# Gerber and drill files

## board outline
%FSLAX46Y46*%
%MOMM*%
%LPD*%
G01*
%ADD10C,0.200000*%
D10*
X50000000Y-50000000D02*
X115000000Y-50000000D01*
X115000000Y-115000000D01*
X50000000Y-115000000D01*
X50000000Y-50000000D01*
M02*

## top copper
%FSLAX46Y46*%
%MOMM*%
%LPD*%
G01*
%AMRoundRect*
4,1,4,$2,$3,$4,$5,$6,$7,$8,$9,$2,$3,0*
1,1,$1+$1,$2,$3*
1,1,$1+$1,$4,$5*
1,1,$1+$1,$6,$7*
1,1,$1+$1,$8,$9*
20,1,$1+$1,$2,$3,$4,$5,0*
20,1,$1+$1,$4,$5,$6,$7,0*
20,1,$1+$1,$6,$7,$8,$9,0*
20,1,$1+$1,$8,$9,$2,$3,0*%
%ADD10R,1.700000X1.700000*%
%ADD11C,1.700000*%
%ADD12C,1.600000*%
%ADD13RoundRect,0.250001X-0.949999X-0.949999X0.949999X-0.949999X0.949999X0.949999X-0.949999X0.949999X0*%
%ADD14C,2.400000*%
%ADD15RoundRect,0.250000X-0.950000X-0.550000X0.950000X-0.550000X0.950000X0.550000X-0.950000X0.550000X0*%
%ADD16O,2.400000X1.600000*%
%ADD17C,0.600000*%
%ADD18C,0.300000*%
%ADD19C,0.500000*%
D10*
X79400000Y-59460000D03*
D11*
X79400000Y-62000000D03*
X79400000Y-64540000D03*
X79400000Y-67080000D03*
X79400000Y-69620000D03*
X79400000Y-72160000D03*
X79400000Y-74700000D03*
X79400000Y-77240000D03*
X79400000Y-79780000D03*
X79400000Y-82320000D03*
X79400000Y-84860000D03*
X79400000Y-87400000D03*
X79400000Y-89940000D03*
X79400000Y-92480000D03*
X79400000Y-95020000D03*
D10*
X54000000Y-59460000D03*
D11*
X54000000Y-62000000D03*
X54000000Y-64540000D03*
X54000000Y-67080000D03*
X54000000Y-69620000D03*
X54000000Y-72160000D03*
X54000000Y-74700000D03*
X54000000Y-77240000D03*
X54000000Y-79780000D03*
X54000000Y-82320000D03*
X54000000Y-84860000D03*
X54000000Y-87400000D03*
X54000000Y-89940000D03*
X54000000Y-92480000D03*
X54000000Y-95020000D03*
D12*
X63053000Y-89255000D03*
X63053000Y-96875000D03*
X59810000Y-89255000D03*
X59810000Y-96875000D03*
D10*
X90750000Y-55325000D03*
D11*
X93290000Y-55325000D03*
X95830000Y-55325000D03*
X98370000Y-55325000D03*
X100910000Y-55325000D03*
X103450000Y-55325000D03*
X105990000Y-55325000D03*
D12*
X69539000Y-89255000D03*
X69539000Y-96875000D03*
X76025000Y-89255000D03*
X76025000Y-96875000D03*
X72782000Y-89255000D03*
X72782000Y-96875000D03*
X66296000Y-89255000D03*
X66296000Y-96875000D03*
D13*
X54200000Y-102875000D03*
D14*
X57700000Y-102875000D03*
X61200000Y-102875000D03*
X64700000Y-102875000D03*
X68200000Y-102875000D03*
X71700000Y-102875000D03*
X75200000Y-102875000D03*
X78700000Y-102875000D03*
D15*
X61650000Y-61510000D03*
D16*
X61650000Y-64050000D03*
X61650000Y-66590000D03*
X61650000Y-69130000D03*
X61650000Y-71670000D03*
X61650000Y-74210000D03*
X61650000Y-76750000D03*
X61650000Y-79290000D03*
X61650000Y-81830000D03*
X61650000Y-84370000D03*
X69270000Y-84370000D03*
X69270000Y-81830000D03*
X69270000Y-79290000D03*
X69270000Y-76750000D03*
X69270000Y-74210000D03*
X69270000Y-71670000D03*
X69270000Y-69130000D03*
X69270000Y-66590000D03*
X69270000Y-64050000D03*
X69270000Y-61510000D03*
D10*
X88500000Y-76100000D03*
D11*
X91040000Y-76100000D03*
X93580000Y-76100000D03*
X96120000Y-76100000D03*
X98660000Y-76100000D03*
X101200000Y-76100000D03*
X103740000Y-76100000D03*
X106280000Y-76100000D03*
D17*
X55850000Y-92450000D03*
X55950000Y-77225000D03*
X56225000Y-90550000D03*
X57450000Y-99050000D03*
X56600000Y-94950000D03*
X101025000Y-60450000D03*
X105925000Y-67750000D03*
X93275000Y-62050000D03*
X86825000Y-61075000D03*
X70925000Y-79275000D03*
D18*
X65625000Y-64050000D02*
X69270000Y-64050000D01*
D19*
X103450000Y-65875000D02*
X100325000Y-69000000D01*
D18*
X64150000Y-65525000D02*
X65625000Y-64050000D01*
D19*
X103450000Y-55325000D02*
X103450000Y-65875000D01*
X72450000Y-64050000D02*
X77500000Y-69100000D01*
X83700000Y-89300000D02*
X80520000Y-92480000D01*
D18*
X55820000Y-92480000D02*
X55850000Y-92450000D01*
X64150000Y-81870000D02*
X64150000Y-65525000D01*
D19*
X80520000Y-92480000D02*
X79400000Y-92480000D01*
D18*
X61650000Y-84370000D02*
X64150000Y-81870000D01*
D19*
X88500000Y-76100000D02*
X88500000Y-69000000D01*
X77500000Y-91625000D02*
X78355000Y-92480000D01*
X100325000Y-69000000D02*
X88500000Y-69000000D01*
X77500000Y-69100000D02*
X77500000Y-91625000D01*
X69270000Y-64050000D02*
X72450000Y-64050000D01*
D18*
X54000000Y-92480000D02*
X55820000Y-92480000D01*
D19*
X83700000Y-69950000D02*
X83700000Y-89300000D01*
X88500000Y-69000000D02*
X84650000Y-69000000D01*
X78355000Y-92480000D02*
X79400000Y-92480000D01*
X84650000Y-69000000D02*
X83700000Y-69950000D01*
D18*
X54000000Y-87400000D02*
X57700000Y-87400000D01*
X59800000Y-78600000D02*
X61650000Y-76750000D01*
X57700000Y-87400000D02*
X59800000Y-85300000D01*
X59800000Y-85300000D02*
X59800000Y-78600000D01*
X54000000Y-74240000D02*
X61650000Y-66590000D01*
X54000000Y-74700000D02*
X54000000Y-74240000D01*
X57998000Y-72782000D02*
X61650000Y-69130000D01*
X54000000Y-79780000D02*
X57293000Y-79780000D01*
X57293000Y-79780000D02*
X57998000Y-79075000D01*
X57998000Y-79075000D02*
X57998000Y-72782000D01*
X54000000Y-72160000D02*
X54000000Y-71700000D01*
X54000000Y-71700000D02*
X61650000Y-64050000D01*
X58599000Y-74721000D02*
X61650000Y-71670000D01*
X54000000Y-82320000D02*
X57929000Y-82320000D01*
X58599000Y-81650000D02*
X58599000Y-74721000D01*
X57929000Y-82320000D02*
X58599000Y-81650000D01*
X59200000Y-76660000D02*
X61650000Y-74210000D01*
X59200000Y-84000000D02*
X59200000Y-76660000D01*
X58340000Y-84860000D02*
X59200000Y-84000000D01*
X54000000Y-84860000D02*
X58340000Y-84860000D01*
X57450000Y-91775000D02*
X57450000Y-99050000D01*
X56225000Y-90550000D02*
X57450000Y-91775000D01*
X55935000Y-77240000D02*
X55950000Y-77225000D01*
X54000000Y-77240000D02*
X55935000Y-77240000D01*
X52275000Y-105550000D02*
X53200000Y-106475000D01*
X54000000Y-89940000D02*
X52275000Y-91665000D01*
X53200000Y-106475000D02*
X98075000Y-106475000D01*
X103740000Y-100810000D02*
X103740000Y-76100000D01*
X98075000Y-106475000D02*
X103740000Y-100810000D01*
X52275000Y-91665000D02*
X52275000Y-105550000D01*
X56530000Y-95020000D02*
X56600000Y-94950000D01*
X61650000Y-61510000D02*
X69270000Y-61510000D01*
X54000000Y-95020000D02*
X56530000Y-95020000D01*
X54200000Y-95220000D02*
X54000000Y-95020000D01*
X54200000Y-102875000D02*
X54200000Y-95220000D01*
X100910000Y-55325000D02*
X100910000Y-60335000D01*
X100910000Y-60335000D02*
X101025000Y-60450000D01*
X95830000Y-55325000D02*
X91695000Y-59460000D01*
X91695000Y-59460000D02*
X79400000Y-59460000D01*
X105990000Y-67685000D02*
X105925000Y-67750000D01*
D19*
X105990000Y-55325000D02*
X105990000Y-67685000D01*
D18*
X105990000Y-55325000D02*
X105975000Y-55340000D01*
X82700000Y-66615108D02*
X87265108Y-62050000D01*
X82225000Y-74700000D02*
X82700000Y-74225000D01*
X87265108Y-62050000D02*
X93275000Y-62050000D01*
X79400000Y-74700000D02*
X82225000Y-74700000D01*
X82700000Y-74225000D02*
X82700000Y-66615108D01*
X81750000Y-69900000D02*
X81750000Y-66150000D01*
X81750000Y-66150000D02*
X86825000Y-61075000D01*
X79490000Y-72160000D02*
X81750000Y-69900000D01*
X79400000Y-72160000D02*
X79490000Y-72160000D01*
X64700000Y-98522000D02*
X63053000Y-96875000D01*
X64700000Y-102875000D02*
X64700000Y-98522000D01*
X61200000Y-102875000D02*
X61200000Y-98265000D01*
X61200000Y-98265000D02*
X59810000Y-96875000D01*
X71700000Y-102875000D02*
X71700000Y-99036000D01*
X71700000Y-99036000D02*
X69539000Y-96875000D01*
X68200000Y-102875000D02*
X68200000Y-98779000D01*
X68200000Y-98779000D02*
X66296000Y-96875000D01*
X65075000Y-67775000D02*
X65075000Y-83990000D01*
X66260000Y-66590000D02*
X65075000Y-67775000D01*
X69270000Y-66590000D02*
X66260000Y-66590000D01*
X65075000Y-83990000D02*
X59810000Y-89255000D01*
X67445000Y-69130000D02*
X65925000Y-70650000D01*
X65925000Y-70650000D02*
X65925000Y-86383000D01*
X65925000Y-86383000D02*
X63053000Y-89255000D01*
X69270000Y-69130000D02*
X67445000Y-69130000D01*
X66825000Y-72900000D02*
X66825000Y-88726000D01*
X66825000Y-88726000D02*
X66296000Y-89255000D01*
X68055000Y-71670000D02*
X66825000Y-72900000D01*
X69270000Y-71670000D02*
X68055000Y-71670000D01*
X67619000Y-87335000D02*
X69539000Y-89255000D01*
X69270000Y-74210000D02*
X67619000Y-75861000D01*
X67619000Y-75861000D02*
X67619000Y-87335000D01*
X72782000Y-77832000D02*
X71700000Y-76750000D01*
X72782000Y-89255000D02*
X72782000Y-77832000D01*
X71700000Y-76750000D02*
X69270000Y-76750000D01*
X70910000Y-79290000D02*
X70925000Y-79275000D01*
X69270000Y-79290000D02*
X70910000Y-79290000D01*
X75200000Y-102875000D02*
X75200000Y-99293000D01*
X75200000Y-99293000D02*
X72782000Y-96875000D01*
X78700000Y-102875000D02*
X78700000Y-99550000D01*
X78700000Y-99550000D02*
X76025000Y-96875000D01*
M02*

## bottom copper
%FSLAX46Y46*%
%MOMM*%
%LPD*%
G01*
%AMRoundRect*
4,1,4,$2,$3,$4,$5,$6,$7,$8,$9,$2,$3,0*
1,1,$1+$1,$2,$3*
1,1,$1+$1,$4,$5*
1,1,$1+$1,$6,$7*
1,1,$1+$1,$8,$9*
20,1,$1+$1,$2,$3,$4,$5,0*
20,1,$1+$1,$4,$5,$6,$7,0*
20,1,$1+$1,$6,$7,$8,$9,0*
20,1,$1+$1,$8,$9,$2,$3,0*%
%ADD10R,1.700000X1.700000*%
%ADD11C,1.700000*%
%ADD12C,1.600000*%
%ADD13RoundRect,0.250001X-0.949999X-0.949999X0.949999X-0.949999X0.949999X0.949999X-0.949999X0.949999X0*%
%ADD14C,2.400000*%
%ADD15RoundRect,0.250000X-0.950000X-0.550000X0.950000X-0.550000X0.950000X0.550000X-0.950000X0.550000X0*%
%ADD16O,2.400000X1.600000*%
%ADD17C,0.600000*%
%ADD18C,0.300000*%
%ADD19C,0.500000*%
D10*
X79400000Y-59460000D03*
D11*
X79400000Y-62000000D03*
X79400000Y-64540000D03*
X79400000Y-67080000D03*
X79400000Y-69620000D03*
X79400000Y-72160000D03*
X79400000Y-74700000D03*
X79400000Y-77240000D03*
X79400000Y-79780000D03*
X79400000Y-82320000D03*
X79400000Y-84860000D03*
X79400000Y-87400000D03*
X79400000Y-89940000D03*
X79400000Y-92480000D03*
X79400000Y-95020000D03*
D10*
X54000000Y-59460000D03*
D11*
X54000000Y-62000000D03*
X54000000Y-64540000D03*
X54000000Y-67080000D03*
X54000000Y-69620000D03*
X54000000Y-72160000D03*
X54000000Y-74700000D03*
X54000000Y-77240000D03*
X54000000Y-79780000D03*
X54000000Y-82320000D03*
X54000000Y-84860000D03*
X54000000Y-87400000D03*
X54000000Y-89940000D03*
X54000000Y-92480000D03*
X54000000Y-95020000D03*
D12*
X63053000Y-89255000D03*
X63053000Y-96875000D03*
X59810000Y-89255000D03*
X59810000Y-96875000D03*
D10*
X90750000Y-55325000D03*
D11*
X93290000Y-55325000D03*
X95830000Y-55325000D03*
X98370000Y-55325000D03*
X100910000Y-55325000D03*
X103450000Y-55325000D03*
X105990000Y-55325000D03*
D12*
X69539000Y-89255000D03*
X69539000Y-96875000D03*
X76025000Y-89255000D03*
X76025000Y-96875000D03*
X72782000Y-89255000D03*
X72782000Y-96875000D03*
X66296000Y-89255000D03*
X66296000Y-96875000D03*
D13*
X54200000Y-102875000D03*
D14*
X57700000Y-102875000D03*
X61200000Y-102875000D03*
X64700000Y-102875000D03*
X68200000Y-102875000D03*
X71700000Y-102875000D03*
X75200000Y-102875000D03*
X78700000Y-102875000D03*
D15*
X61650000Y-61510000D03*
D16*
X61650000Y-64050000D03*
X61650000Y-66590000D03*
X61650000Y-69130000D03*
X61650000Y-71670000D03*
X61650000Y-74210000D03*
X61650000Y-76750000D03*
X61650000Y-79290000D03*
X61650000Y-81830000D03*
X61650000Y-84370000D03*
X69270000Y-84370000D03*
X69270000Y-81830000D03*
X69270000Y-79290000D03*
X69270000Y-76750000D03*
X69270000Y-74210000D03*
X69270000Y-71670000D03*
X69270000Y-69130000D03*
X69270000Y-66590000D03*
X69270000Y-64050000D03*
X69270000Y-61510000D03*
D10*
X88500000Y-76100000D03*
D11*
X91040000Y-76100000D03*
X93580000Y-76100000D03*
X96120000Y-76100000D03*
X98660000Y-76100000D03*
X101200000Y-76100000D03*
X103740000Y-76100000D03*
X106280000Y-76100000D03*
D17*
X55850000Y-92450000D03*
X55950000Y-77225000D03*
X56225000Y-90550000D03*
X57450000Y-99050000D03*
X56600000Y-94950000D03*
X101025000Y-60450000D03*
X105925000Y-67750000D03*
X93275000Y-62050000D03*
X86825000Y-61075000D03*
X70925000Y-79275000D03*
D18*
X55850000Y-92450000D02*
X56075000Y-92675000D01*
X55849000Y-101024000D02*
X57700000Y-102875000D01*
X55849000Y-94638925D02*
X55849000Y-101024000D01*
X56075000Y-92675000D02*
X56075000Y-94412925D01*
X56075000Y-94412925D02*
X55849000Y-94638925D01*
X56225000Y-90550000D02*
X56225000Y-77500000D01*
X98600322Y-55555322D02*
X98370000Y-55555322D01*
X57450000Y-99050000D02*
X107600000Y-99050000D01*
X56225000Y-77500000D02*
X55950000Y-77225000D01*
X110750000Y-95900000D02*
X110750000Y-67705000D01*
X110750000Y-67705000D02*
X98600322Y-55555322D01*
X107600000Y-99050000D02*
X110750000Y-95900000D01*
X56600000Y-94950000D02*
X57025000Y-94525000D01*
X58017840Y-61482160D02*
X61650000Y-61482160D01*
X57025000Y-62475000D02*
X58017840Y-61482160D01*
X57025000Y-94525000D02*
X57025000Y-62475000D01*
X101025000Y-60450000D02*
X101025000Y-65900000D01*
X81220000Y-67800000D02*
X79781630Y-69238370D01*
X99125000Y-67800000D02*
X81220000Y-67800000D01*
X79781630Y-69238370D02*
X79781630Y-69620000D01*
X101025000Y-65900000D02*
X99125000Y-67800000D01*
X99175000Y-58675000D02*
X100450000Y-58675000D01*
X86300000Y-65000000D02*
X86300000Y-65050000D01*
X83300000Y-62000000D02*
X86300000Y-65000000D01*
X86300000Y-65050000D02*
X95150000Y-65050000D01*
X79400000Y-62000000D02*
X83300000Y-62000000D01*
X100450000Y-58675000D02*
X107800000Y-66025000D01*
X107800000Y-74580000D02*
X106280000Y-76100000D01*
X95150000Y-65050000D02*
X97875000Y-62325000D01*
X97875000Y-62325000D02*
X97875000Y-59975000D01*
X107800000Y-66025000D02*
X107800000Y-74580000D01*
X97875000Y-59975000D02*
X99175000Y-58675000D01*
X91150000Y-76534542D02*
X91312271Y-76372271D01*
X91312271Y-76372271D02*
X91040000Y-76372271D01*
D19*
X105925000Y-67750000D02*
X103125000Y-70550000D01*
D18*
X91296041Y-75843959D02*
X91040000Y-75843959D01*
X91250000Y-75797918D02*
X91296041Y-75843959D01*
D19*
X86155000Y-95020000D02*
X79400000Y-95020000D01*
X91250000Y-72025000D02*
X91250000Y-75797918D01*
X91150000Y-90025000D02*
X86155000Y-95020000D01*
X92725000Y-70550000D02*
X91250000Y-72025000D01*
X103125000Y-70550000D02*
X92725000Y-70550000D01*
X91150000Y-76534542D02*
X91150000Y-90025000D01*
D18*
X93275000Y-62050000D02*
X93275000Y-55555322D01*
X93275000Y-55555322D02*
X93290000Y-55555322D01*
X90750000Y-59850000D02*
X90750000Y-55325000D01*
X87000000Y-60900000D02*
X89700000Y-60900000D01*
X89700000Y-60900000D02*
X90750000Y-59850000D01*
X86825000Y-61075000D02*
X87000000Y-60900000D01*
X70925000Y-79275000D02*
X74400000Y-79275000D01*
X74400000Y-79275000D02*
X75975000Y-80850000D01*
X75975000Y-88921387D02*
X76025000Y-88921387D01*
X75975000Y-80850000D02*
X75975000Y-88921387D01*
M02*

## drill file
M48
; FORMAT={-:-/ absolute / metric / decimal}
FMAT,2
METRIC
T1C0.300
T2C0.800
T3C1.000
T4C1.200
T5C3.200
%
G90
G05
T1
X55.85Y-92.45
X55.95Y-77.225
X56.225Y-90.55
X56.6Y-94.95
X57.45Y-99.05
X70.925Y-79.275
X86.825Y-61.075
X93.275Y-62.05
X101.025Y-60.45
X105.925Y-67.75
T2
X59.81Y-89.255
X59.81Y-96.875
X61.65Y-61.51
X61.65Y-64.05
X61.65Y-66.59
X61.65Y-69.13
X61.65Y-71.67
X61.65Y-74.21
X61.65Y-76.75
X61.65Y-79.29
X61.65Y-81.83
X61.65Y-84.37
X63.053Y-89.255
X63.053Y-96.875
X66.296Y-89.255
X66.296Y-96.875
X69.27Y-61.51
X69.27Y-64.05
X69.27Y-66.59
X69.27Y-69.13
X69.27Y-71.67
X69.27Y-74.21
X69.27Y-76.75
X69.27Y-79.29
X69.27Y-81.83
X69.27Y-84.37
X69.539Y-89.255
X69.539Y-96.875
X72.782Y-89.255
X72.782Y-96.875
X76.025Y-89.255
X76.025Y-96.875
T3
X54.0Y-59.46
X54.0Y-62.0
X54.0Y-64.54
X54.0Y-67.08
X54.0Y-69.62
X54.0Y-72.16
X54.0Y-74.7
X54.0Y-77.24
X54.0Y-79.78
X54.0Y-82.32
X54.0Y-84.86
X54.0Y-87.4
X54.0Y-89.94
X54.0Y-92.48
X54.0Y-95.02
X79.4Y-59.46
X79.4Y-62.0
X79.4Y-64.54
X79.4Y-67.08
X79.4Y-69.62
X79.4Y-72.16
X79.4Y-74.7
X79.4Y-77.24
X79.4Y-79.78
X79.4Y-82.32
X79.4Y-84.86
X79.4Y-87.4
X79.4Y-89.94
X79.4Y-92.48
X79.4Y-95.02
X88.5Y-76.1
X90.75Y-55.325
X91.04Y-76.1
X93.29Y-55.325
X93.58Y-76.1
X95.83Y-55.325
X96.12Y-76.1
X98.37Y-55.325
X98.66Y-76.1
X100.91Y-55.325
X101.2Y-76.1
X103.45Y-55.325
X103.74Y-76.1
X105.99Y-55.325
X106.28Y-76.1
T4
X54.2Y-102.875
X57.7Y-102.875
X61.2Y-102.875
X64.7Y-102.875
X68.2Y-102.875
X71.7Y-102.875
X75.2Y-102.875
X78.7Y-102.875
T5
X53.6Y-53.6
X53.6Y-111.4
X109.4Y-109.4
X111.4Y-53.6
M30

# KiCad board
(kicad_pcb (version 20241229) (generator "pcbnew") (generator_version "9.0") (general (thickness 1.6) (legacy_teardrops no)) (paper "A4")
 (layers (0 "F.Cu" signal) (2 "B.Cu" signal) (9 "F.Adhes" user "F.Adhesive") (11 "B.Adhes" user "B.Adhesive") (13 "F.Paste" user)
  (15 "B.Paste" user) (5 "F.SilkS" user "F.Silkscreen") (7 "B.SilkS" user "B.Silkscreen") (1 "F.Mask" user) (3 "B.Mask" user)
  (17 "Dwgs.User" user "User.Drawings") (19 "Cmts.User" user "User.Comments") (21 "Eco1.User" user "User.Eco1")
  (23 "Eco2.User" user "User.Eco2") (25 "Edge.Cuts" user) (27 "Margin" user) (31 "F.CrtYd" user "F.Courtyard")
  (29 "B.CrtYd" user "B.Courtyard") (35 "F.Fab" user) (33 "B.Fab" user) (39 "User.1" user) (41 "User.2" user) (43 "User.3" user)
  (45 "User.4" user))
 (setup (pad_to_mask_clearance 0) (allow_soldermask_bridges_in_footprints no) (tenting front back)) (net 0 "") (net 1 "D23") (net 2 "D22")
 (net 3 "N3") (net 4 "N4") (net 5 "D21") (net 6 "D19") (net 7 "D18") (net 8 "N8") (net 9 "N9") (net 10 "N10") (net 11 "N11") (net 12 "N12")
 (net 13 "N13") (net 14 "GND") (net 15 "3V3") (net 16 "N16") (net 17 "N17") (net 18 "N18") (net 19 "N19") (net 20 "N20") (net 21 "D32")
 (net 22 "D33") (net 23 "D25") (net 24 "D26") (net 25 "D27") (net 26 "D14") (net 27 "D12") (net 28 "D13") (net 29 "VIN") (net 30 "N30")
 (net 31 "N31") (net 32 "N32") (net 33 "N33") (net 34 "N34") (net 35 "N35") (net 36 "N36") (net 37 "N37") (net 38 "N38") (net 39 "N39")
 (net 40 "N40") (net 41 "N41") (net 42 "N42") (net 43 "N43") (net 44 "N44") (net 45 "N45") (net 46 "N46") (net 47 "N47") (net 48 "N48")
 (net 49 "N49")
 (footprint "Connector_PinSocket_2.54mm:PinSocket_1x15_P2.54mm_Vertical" (layer "F.Cu") (at 79.4 59.46)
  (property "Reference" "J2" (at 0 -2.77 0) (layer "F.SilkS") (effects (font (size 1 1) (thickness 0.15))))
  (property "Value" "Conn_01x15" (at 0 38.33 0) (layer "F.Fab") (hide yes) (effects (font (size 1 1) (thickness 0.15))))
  (pad "1" thru_hole rect (at 0 0) (size 1.7 1.7) (drill 1) (layers "*.Cu" "*.Mask") (remove_unused_layers no) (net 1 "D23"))
  (pad "2" thru_hole circle (at 0 2.54) (size 1.7 1.7) (drill 1) (layers "*.Cu" "*.Mask") (remove_unused_layers no) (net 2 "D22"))
  (pad "3" thru_hole circle (at 0 5.08) (size 1.7 1.7) (drill 1) (layers "*.Cu" "*.Mask") (remove_unused_layers no) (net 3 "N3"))
  (pad "4" thru_hole circle (at 0 7.62) (size 1.7 1.7) (drill 1) (layers "*.Cu" "*.Mask") (remove_unused_layers no) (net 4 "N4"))
  (pad "5" thru_hole circle (at 0 10.16) (size 1.7 1.7) (drill 1) (layers "*.Cu" "*.Mask") (remove_unused_layers no) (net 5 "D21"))
  (pad "6" thru_hole circle (at 0 12.7) (size 1.7 1.7) (drill 1) (layers "*.Cu" "*.Mask") (remove_unused_layers no) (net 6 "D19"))
  (pad "7" thru_hole circle (at 0 15.24) (size 1.7 1.7) (drill 1) (layers "*.Cu" "*.Mask") (remove_unused_layers no) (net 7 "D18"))
  (pad "8" thru_hole circle (at 0 17.78) (size 1.7 1.7) (drill 1) (layers "*.Cu" "*.Mask") (remove_unused_layers no) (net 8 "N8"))
  (pad "9" thru_hole circle (at 0 20.32) (size 1.7 1.7) (drill 1) (layers "*.Cu" "*.Mask") (remove_unused_layers no) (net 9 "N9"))
  (pad "10" thru_hole circle (at 0 22.86) (size 1.7 1.7) (drill 1) (layers "*.Cu" "*.Mask") (remove_unused_layers no) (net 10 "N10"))
  (pad "11" thru_hole circle (at 0 25.4) (size 1.7 1.7) (drill 1) (layers "*.Cu" "*.Mask") (remove_unused_layers no) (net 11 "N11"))
  (pad "12" thru_hole circle (at 0 27.94) (size 1.7 1.7) (drill 1) (layers "*.Cu" "*.Mask") (remove_unused_layers no) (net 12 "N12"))
  (pad "13" thru_hole circle (at 0 30.48) (size 1.7 1.7) (drill 1) (layers "*.Cu" "*.Mask") (remove_unused_layers no) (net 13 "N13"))
  (pad "14" thru_hole circle (at 0 33.02) (size 1.7 1.7) (drill 1) (layers "*.Cu" "*.Mask") (remove_unused_layers no) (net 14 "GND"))
  (pad "15" thru_hole circle (at 0 35.56) (size 1.7 1.7) (drill 1) (layers "*.Cu" "*.Mask") (remove_unused_layers no) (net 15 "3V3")))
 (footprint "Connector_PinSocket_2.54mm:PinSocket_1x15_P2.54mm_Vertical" (layer "F.Cu") (at 54 59.46)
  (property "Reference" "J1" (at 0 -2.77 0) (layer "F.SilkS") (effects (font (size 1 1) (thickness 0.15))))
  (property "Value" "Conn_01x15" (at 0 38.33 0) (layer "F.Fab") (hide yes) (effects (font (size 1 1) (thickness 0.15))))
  (pad "1" thru_hole rect (at 0 0) (size 1.7 1.7) (drill 1) (layers "*.Cu" "*.Mask") (remove_unused_layers no) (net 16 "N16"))
  (pad "2" thru_hole circle (at 0 2.54) (size 1.7 1.7) (drill 1) (layers "*.Cu" "*.Mask") (remove_unused_layers no) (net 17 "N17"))
  (pad "3" thru_hole circle (at 0 5.08) (size 1.7 1.7) (drill 1) (layers "*.Cu" "*.Mask") (remove_unused_layers no) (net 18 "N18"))
  (pad "4" thru_hole circle (at 0 7.62) (size 1.7 1.7) (drill 1) (layers "*.Cu" "*.Mask") (remove_unused_layers no) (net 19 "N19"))
  (pad "5" thru_hole circle (at 0 10.16) (size 1.7 1.7) (drill 1) (layers "*.Cu" "*.Mask") (remove_unused_layers no) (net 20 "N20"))
  (pad "6" thru_hole circle (at 0 12.7) (size 1.7 1.7) (drill 1) (layers "*.Cu" "*.Mask") (remove_unused_layers no) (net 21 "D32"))
  (pad "7" thru_hole circle (at 0 15.24) (size 1.7 1.7) (drill 1) (layers "*.Cu" "*.Mask") (remove_unused_layers no) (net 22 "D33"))
  (pad "8" thru_hole circle (at 0 17.78) (size 1.7 1.7) (drill 1) (layers "*.Cu" "*.Mask") (remove_unused_layers no) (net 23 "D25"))
  (pad "9" thru_hole circle (at 0 20.32) (size 1.7 1.7) (drill 1) (layers "*.Cu" "*.Mask") (remove_unused_layers no) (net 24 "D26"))
  (pad "10" thru_hole circle (at 0 22.86) (size 1.7 1.7) (drill 1) (layers "*.Cu" "*.Mask") (remove_unused_layers no) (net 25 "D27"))
  (pad "11" thru_hole circle (at 0 25.4) (size 1.7 1.7) (drill 1) (layers "*.Cu" "*.Mask") (remove_unused_layers no) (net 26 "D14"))
  (pad "12" thru_hole circle (at 0 27.94) (size 1.7 1.7) (drill 1) (layers "*.Cu" "*.Mask") (remove_unused_layers no) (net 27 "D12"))
  (pad "13" thru_hole circle (at 0 30.48) (size 1.7 1.7) (drill 1) (layers "*.Cu" "*.Mask") (remove_unused_layers no) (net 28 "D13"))
  (pad "14" thru_hole circle (at 0 33.02) (size 1.7 1.7) (drill 1) (layers "*.Cu" "*.Mask") (remove_unused_layers no) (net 14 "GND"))
  (pad "15" thru_hole circle (at 0 35.56) (size 1.7 1.7) (drill 1) (layers "*.Cu" "*.Mask") (remove_unused_layers no) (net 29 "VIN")))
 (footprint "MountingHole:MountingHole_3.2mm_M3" (layer "F.Cu") (at 53.6 53.6)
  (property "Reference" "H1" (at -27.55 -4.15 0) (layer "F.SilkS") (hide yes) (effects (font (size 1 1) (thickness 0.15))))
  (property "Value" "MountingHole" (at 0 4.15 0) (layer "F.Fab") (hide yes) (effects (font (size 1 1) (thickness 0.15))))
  (pad "" np_thru_hole circle (at 0 0) (size 3.2 3.2) (drill 3.2) (layers "*.Cu" "*.Mask")))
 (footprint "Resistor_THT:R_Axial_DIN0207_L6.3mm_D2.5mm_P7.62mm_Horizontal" (layer "F.Cu") (at 63.053 89.255 -90)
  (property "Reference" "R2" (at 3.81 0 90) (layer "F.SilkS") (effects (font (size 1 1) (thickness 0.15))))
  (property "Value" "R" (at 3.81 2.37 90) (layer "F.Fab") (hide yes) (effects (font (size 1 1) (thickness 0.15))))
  (pad "1" thru_hole circle (at 0 0 270) (size 1.6 1.6) (drill 0.8) (layers "*.Cu" "*.Mask") (remove_unused_layers no) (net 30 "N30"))
  (pad "2" thru_hole circle (at 7.62 0 270) (size 1.6 1.6) (drill 0.8) (layers "*.Cu" "*.Mask") (remove_unused_layers no) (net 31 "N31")))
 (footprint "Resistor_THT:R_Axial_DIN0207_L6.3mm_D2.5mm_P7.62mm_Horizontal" (layer "F.Cu") (at 59.81 89.255 -90)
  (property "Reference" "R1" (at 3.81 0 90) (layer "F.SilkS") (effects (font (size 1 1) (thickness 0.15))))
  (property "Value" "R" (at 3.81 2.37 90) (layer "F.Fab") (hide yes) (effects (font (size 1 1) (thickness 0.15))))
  (pad "1" thru_hole circle (at 0 0 270) (size 1.6 1.6) (drill 0.8) (layers "*.Cu" "*.Mask") (remove_unused_layers no) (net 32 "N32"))
  (pad "2" thru_hole circle (at 7.62 0 270) (size 1.6 1.6) (drill 0.8) (layers "*.Cu" "*.Mask") (remove_unused_layers no) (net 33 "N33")))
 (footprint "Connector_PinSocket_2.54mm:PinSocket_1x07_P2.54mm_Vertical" (layer "F.Cu") (at 90.75 55.325 90)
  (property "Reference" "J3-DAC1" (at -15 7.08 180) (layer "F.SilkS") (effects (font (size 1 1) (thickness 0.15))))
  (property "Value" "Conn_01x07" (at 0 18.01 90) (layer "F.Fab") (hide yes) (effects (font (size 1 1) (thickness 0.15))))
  (pad "1" thru_hole rect (at 0 0 90) (size 1.7 1.7) (drill 1) (layers "*.Cu" "*.Mask") (remove_unused_layers no) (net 6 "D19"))
  (pad "2" thru_hole circle (at 0 2.54 90) (size 1.7 1.7) (drill 1) (layers "*.Cu" "*.Mask") (remove_unused_layers no) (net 7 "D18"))
  (pad "3" thru_hole circle (at 0 5.08 90) (size 1.7 1.7) (drill 1) (layers "*.Cu" "*.Mask") (remove_unused_layers no) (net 1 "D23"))
  (pad "4" thru_hole circle (at 0 7.62 90) (size 1.7 1.7) (drill 1) (layers "*.Cu" "*.Mask") (remove_unused_layers no) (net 23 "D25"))
  (pad "5" thru_hole circle (at 0 10.16 90) (size 1.7 1.7) (drill 1) (layers "*.Cu" "*.Mask") (remove_unused_layers no) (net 5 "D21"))
  (pad "6" thru_hole circle (at 0 12.7 90) (size 1.7 1.7) (drill 1) (layers "*.Cu" "*.Mask") (remove_unused_layers no) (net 14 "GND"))
  (pad "7" thru_hole circle (at 0 15.24 90) (size 1.7 1.7) (drill 1) (layers "*.Cu" "*.Mask") (remove_unused_layers no) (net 15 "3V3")))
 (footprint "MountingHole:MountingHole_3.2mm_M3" (layer "F.Cu") (at 53.6 111.4)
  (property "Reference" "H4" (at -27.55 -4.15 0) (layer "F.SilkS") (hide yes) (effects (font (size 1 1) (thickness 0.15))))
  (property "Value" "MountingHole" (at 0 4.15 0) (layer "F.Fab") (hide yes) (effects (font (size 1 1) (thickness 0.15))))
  (pad "" np_thru_hole circle (at 0 0) (size 3.2 3.2) (drill 3.2) (layers "*.Cu" "*.Mask")))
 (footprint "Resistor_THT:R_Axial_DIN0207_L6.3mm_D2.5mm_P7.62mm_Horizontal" (layer "F.Cu") (at 69.539 89.255 -90)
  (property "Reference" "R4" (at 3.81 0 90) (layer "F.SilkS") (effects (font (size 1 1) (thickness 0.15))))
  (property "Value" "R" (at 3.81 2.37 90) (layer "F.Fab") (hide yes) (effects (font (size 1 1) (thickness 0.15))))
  (pad "1" thru_hole circle (at 0 0 270) (size 1.6 1.6) (drill 0.8) (layers "*.Cu" "*.Mask") (remove_unused_layers no) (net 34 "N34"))
  (pad "2" thru_hole circle (at 7.62 0 270) (size 1.6 1.6) (drill 0.8) (layers "*.Cu" "*.Mask") (remove_unused_layers no) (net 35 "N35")))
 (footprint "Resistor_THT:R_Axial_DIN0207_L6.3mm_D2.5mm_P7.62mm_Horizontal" (layer "F.Cu") (at 76.025 89.255 -90)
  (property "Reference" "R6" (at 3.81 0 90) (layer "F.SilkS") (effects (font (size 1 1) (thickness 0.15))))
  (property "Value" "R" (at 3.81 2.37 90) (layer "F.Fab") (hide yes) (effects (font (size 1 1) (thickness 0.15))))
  (pad "1" thru_hole circle (at 0 0 270) (size 1.6 1.6) (drill 0.8) (layers "*.Cu" "*.Mask") (remove_unused_layers no) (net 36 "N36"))
  (pad "2" thru_hole circle (at 7.62 0 270) (size 1.6 1.6) (drill 0.8) (layers "*.Cu" "*.Mask") (remove_unused_layers no) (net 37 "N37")))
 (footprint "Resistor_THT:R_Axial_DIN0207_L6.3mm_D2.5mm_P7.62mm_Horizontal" (layer "F.Cu") (at 72.782 89.255 -90)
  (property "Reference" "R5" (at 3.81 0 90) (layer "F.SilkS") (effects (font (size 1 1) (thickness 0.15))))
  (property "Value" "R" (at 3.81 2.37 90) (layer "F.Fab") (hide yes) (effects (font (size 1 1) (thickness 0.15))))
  (pad "1" thru_hole circle (at 0 0 270) (size 1.6 1.6) (drill 0.8) (layers "*.Cu" "*.Mask") (remove_unused_layers no) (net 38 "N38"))
  (pad "2" thru_hole circle (at 7.62 0 270) (size 1.6 1.6) (drill 0.8) (layers "*.Cu" "*.Mask") (remove_unused_layers no) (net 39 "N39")))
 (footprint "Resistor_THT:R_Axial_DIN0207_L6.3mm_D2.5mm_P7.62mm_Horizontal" (layer "F.Cu") (at 66.296 89.255 -90)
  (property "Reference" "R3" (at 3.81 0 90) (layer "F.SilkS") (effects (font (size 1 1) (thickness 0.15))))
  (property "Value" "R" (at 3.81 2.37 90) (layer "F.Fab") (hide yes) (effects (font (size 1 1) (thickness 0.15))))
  (pad "1" thru_hole circle (at 0 0 270) (size 1.6 1.6) (drill 0.8) (layers "*.Cu" "*.Mask") (remove_unused_layers no) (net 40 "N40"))
  (pad "2" thru_hole circle (at 7.62 0 270) (size 1.6 1.6) (drill 0.8) (layers "*.Cu" "*.Mask") (remove_unused_layers no) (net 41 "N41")))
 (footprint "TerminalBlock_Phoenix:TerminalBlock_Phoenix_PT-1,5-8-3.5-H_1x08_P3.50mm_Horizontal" (layer "F.Cu") (at 54.2 102.875)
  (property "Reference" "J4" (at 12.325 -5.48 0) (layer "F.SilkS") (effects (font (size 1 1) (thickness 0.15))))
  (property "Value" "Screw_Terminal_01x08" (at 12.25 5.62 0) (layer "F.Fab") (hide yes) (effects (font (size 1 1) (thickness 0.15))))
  (pad "1" thru_hole roundrect (at 0 0) (size 2.4 2.4) (drill 1.2) (layers "*.Cu" "*.Mask") (remove_unused_layers no)
   (roundrect_rratio 0.104167) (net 29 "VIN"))
  (pad "2" thru_hole circle (at 3.5 0) (size 2.4 2.4) (drill 1.2) (layers "*.Cu" "*.Mask") (remove_unused_layers no) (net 14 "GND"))
  (pad "3" thru_hole circle (at 7 0) (size 2.4 2.4) (drill 1.2) (layers "*.Cu" "*.Mask") (remove_unused_layers no) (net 33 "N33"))
  (pad "4" thru_hole circle (at 10.5 0) (size 2.4 2.4) (drill 1.2) (layers "*.Cu" "*.Mask") (remove_unused_layers no) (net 31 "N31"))
  (pad "5" thru_hole circle (at 14 0) (size 2.4 2.4) (drill 1.2) (layers "*.Cu" "*.Mask") (remove_unused_layers no) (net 41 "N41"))
  (pad "6" thru_hole circle (at 17.5 0) (size 2.4 2.4) (drill 1.2) (layers "*.Cu" "*.Mask") (remove_unused_layers no) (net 35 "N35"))
  (pad "7" thru_hole circle (at 21 0) (size 2.4 2.4) (drill 1.2) (layers "*.Cu" "*.Mask") (remove_unused_layers no) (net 39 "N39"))
  (pad "8" thru_hole circle (at 24.5 0) (size 2.4 2.4) (drill 1.2) (layers "*.Cu" "*.Mask") (remove_unused_layers no) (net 37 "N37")))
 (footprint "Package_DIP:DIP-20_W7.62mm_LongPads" (layer "F.Cu") (at 61.65 61.51)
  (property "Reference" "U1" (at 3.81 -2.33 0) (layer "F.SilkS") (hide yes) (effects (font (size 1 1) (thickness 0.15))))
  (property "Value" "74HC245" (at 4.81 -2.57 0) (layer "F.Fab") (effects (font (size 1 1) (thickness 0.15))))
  (pad "1" thru_hole roundrect (at 0 0) (size 2.4 1.6) (drill 0.8) (layers "*.Cu" "*.Mask") (remove_unused_layers no)
   (roundrect_rratio 0.15625) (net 29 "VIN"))
  (pad "2" thru_hole oval (at 0 2.54) (size 2.4 1.6) (drill 0.8) (layers "*.Cu" "*.Mask") (remove_unused_layers no) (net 21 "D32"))
  (pad "3" thru_hole oval (at 0 5.08) (size 2.4 1.6) (drill 0.8) (layers "*.Cu" "*.Mask") (remove_unused_layers no) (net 22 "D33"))
  (pad "4" thru_hole oval (at 0 7.62) (size 2.4 1.6) (drill 0.8) (layers "*.Cu" "*.Mask") (remove_unused_layers no) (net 24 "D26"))
  (pad "5" thru_hole oval (at 0 10.16) (size 2.4 1.6) (drill 0.8) (layers "*.Cu" "*.Mask") (remove_unused_layers no) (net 25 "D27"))
  (pad "6" thru_hole oval (at 0 12.7) (size 2.4 1.6) (drill 0.8) (layers "*.Cu" "*.Mask") (remove_unused_layers no) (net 26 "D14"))
  (pad "7" thru_hole oval (at 0 15.24) (size 2.4 1.6) (drill 0.8) (layers "*.Cu" "*.Mask") (remove_unused_layers no) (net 27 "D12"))
  (pad "8" thru_hole oval (at 0 17.78) (size 2.4 1.6) (drill 0.8) (layers "*.Cu" "*.Mask") (remove_unused_layers no) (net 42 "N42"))
  (pad "9" thru_hole oval (at 0 20.32) (size 2.4 1.6) (drill 0.8) (layers "*.Cu" "*.Mask") (remove_unused_layers no) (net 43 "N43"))
  (pad "10" thru_hole oval (at 0 22.86) (size 2.4 1.6) (drill 0.8) (layers "*.Cu" "*.Mask") (remove_unused_layers no) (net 14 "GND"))
  (pad "11" thru_hole oval (at 7.62 22.86) (size 2.4 1.6) (drill 0.8) (layers "*.Cu" "*.Mask") (remove_unused_layers no) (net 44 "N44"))
  (pad "12" thru_hole oval (at 7.62 20.32) (size 2.4 1.6) (drill 0.8) (layers "*.Cu" "*.Mask") (remove_unused_layers no) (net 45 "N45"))
  (pad "13" thru_hole oval (at 7.62 17.78) (size 2.4 1.6) (drill 0.8) (layers "*.Cu" "*.Mask") (remove_unused_layers no) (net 36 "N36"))
  (pad "14" thru_hole oval (at 7.62 15.24) (size 2.4 1.6) (drill 0.8) (layers "*.Cu" "*.Mask") (remove_unused_layers no) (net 38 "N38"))
  (pad "15" thru_hole oval (at 7.62 12.7) (size 2.4 1.6) (drill 0.8) (layers "*.Cu" "*.Mask") (remove_unused_layers no) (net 34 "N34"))
  (pad "16" thru_hole oval (at 7.62 10.16) (size 2.4 1.6) (drill 0.8) (layers "*.Cu" "*.Mask") (remove_unused_layers no) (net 40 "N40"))
  (pad "17" thru_hole oval (at 7.62 7.62) (size 2.4 1.6) (drill 0.8) (layers "*.Cu" "*.Mask") (remove_unused_layers no) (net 30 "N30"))
  (pad "18" thru_hole oval (at 7.62 5.08) (size 2.4 1.6) (drill 0.8) (layers "*.Cu" "*.Mask") (remove_unused_layers no) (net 32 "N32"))
  (pad "19" thru_hole oval (at 7.62 2.54) (size 2.4 1.6) (drill 0.8) (layers "*.Cu" "*.Mask") (remove_unused_layers no) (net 14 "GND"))
  (pad "20" thru_hole oval (at 7.62 0) (size 2.4 1.6) (drill 0.8) (layers "*.Cu" "*.Mask") (remove_unused_layers no) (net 29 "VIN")))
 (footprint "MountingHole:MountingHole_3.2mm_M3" (layer "F.Cu") (at 109.4 109.4)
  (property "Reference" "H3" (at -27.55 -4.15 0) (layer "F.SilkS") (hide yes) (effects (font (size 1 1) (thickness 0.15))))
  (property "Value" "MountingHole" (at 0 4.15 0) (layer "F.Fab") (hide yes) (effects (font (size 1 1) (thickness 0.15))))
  (pad "" np_thru_hole circle (at 0 0) (size 3.2 3.2) (drill 3.2) (layers "*.Cu" "*.Mask")))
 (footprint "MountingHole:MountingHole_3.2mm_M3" (layer "F.Cu") (at 111.4 53.6)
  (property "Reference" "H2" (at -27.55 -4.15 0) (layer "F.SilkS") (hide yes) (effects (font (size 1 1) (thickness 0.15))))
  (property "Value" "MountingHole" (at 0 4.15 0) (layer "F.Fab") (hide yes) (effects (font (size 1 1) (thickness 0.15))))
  (pad "" np_thru_hole circle (at 0 0) (size 3.2 3.2) (drill 3.2) (layers "*.Cu" "*.Mask")))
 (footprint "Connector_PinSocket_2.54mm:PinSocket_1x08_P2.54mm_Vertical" (layer "F.Cu") (at 88.5 76.1 90)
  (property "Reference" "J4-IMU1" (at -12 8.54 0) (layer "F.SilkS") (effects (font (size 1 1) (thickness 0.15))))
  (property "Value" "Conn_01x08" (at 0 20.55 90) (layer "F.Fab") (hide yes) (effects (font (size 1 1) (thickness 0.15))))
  (pad "1" thru_hole rect (at 0 0 90) (size 1.7 1.7) (drill 1) (layers "*.Cu" "*.Mask") (remove_unused_layers no) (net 14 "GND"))
  (pad "2" thru_hole circle (at 0 2.54 90) (size 1.7 1.7) (drill 1) (layers "*.Cu" "*.Mask") (remove_unused_layers no) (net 15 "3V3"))
  (pad "3" thru_hole circle (at 0 5.08 90) (size 1.7 1.7) (drill 1) (layers "*.Cu" "*.Mask") (remove_unused_layers no) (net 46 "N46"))
  (pad "4" thru_hole circle (at 0 7.62 90) (size 1.7 1.7) (drill 1) (layers "*.Cu" "*.Mask") (remove_unused_layers no) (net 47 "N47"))
  (pad "5" thru_hole circle (at 0 10.16 90) (size 1.7 1.7) (drill 1) (layers "*.Cu" "*.Mask") (remove_unused_layers no) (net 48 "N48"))
  (pad "6" thru_hole circle (at 0 12.7 90) (size 1.7 1.7) (drill 1) (layers "*.Cu" "*.Mask") (remove_unused_layers no) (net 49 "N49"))
  (pad "7" thru_hole circle (at 0 15.24 90) (size 1.7 1.7) (drill 1) (layers "*.Cu" "*.Mask") (remove_unused_layers no) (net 28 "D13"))
  (pad "8" thru_hole circle (at 0 17.78 90) (size 1.7 1.7) (drill 1) (layers "*.Cu" "*.Mask") (remove_unused_layers no) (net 2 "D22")))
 (gr_rect (start 50 50) (end 115 115) (stroke (width 0.2) (type solid)) (fill no) (layer "Edge.Cuts"))
 (segment (start 65.625 64.05) (end 69.27 64.05) (width 0.3) (layer "F.Cu") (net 14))
 (segment (start 103.45 65.875) (end 100.325 69) (width 0.5) (layer "F.Cu") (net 14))
 (segment (start 64.15 65.525) (end 65.625 64.05) (width 0.3) (layer "F.Cu") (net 14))
 (segment (start 103.45 55.325) (end 103.45 65.875) (width 0.5) (layer "F.Cu") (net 14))
 (segment (start 72.45 64.05) (end 77.5 69.1) (width 0.5) (layer "F.Cu") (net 14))
 (segment (start 83.7 89.3) (end 80.52 92.48) (width 0.5) (layer "F.Cu") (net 14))
 (segment (start 55.82 92.48) (end 55.85 92.45) (width 0.3) (layer "F.Cu") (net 14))
 (segment (start 64.15 81.87) (end 64.15 65.525) (width 0.3) (layer "F.Cu") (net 14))
 (segment (start 80.52 92.48) (end 79.4 92.48) (width 0.5) (layer "F.Cu") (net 14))
 (segment (start 61.65 84.37) (end 64.15 81.87) (width 0.3) (layer "F.Cu") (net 14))
 (segment (start 88.5 76.1) (end 88.5 69) (width 0.5) (layer "F.Cu") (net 14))
 (segment (start 77.5 91.625) (end 78.355 92.48) (width 0.5) (layer "F.Cu") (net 14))
 (segment (start 100.325 69) (end 88.5 69) (width 0.5) (layer "F.Cu") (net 14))
 (segment (start 77.5 69.1) (end 77.5 91.625) (width 0.5) (layer "F.Cu") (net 14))
 (segment (start 69.27 64.05) (end 72.45 64.05) (width 0.5) (layer "F.Cu") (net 14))
 (segment (start 54 92.48) (end 55.82 92.48) (width 0.3) (layer "F.Cu") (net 14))
 (segment (start 83.7 69.95) (end 83.7 89.3) (width 0.5) (layer "F.Cu") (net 14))
 (segment (start 88.5 69) (end 84.65 69) (width 0.5) (layer "F.Cu") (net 14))
 (segment (start 78.355 92.48) (end 79.4 92.48) (width 0.5) (layer "F.Cu") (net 14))
 (segment (start 84.65 69) (end 83.7 69.95) (width 0.5) (layer "F.Cu") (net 14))
 (via (at 55.85 92.45) (size 0.6) (drill 0.3) (layers "F.Cu" "B.Cu") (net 14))
 (segment (start 55.85 92.45) (end 56.075 92.675) (width 0.3) (layer "B.Cu") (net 14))
 (segment (start 55.849 101.024) (end 57.7 102.875) (width 0.3) (layer "B.Cu") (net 14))
 (segment (start 55.849 94.638925) (end 55.849 101.024) (width 0.3) (layer "B.Cu") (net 14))
 (segment (start 56.075 92.675) (end 56.075 94.412925) (width 0.3) (layer "B.Cu") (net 14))
 (segment (start 56.075 94.412925) (end 55.849 94.638925) (width 0.3) (layer "B.Cu") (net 14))
 (segment (start 54 87.4) (end 57.7 87.4) (width 0.3) (layer "F.Cu") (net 27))
 (segment (start 59.8 78.6) (end 61.65 76.75) (width 0.3) (layer "F.Cu") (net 27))
 (segment (start 57.7 87.4) (end 59.8 85.3) (width 0.3) (layer "F.Cu") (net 27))
 (segment (start 59.8 85.3) (end 59.8 78.6) (width 0.3) (layer "F.Cu") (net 27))
 (segment (start 54 74.24) (end 61.65 66.59) (width 0.3) (layer "F.Cu") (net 22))
 (segment (start 54 74.7) (end 54 74.24) (width 0.3) (layer "F.Cu") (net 22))
 (segment (start 57.998 72.782) (end 61.65 69.13) (width 0.3) (layer "F.Cu") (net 24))
 (segment (start 54 79.78) (end 57.293 79.78) (width 0.3) (layer "F.Cu") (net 24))
 (segment (start 57.293 79.78) (end 57.998 79.075) (width 0.3) (layer "F.Cu") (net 24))
 (segment (start 57.998 79.075) (end 57.998 72.782) (width 0.3) (layer "F.Cu") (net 24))
 (segment (start 54 72.16) (end 54 71.7) (width 0.3) (layer "F.Cu") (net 21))
 (segment (start 54 71.7) (end 61.65 64.05) (width 0.3) (layer "F.Cu") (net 21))
 (segment (start 58.599 74.721) (end 61.65 71.67) (width 0.3) (layer "F.Cu") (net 25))
 (segment (start 54 82.32) (end 57.929 82.32) (width 0.3) (layer "F.Cu") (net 25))
 (segment (start 58.599 81.65) (end 58.599 74.721) (width 0.3) (layer "F.Cu") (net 25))
 (segment (start 57.929 82.32) (end 58.599 81.65) (width 0.3) (layer "F.Cu") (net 25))
 (segment (start 59.2 76.66) (end 61.65 74.21) (width 0.3) (layer "F.Cu") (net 26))
 (segment (start 59.2 84) (end 59.2 76.66) (width 0.3) (layer "F.Cu") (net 26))
 (segment (start 58.34 84.86) (end 59.2 84) (width 0.3) (layer "F.Cu") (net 26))
 (segment (start 54 84.86) (end 58.34 84.86) (width 0.3) (layer "F.Cu") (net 26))
 (segment (start 57.45 91.775) (end 57.45 99.05) (width 0.3) (layer "F.Cu") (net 23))
 (segment (start 56.225 90.55) (end 57.45 91.775) (width 0.3) (layer "F.Cu") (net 23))
 (segment (start 55.935 77.24) (end 55.95 77.225) (width 0.3) (layer "F.Cu") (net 23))
 (segment (start 54 77.24) (end 55.935 77.24) (width 0.3) (layer "F.Cu") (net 23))
 (via (at 55.95 77.225) (size 0.6) (drill 0.3) (layers "F.Cu" "B.Cu") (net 23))
 (via (at 56.225 90.55) (size 0.6) (drill 0.3) (layers "F.Cu" "B.Cu") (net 23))
 (via (at 57.45 99.05) (size 0.6) (drill 0.3) (layers "F.Cu" "B.Cu") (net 23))
 (segment (start 56.225 90.55) (end 56.225 77.5) (width 0.3) (layer "B.Cu") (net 23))
 (segment (start 98.600322 55.555322) (end 98.37 55.555322) (width 0.3) (layer "B.Cu") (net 23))
 (segment (start 57.45 99.05) (end 107.6 99.05) (width 0.3) (layer "B.Cu") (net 23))
 (segment (start 56.225 77.5) (end 55.95 77.225) (width 0.3) (layer "B.Cu") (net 23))
 (segment (start 110.75 95.9) (end 110.75 67.705) (width 0.3) (layer "B.Cu") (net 23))
 (segment (start 110.75 67.705) (end 98.600322 55.555322) (width 0.3) (layer "B.Cu") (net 23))
 (segment (start 107.6 99.05) (end 110.75 95.9) (width 0.3) (layer "B.Cu") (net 23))
 (segment (start 52.275 105.55) (end 53.2 106.475) (width 0.3) (layer "F.Cu") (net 28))
 (segment (start 54 89.94) (end 52.275 91.665) (width 0.3) (layer "F.Cu") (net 28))
 (segment (start 53.2 106.475) (end 98.075 106.475) (width 0.3) (layer "F.Cu") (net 28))
 (segment (start 103.74 100.81) (end 103.74 76.1) (width 0.3) (layer "F.Cu") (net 28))
 (segment (start 98.075 106.475) (end 103.74 100.81) (width 0.3) (layer "F.Cu") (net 28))
 (segment (start 52.275 91.665) (end 52.275 105.55) (width 0.3) (layer "F.Cu") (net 28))
 (segment (start 56.53 95.02) (end 56.6 94.95) (width 0.3) (layer "F.Cu") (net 29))
 (segment (start 61.65 61.51) (end 69.27 61.51) (width 0.3) (layer "F.Cu") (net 29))
 (segment (start 54 95.02) (end 56.53 95.02) (width 0.3) (layer "F.Cu") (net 29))
 (segment (start 54.2 95.22) (end 54 95.02) (width 0.3) (layer "F.Cu") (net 29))
 (segment (start 54.2 102.875) (end 54.2 95.22) (width 0.3) (layer "F.Cu") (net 29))
 (via (at 56.6 94.95) (size 0.6) (drill 0.3) (layers "F.Cu" "B.Cu") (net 29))
 (segment (start 56.6 94.95) (end 57.025 94.525) (width 0.3) (layer "B.Cu") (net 29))
 (segment (start 58.01784 61.48216) (end 61.65 61.48216) (width 0.3) (layer "B.Cu") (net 29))
 (segment (start 57.025 62.475) (end 58.01784 61.48216) (width 0.3) (layer "B.Cu") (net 29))
 (segment (start 57.025 94.525) (end 57.025 62.475) (width 0.3) (layer "B.Cu") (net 29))
 (segment (start 100.91 55.325) (end 100.91 60.335) (width 0.3) (layer "F.Cu") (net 5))
 (segment (start 100.91 60.335) (end 101.025 60.45) (width 0.3) (layer "F.Cu") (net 5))
 (via (at 101.025 60.45) (size 0.6) (drill 0.3) (layers "F.Cu" "B.Cu") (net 5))
 (segment (start 101.025 60.45) (end 101.025 65.9) (width 0.3) (layer "B.Cu") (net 5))
 (segment (start 81.22 67.8) (end 79.78163 69.23837) (width 0.3) (layer "B.Cu") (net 5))
 (segment (start 99.125 67.8) (end 81.22 67.8) (width 0.3) (layer "B.Cu") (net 5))
 (segment (start 79.78163 69.23837) (end 79.78163 69.62) (width 0.3) (layer "B.Cu") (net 5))
 (segment (start 101.025 65.9) (end 99.125 67.8) (width 0.3) (layer "B.Cu") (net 5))
 (segment (start 95.83 55.325) (end 91.695 59.46) (width 0.3) (layer "F.Cu") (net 1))
 (segment (start 91.695 59.46) (end 79.4 59.46) (width 0.3) (layer "F.Cu") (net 1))
 (segment (start 99.175 58.675) (end 100.45 58.675) (width 0.3) (layer "B.Cu") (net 2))
 (segment (start 86.3 65) (end 86.3 65.05) (width 0.3) (layer "B.Cu") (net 2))
 (segment (start 83.3 62) (end 86.3 65) (width 0.3) (layer "B.Cu") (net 2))
 (segment (start 86.3 65.05) (end 95.15 65.05) (width 0.3) (layer "B.Cu") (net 2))
 (segment (start 79.4 62) (end 83.3 62) (width 0.3) (layer "B.Cu") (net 2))
 (segment (start 100.45 58.675) (end 107.8 66.025) (width 0.3) (layer "B.Cu") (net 2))
 (segment (start 107.8 74.58) (end 106.28 76.1) (width 0.3) (layer "B.Cu") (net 2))
 (segment (start 95.15 65.05) (end 97.875 62.325) (width 0.3) (layer "B.Cu") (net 2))
 (segment (start 97.875 62.325) (end 97.875 59.975) (width 0.3) (layer "B.Cu") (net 2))
 (segment (start 107.8 66.025) (end 107.8 74.58) (width 0.3) (layer "B.Cu") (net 2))
 (segment (start 97.875 59.975) (end 99.175 58.675) (width 0.3) (layer "B.Cu") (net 2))
 (segment (start 105.99 67.685) (end 105.925 67.75) (width 0.3) (layer "F.Cu") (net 15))
 (segment (start 105.99 55.325) (end 105.99 67.685) (width 0.5) (layer "F.Cu") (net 15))
 (segment (start 105.99 55.325) (end 105.975 55.34) (width 0.3) (layer "F.Cu") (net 15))
 (via (at 105.925 67.75) (size 0.6) (drill 0.3) (layers "F.Cu" "B.Cu") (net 15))
 (segment (start 91.15 76.534542) (end 91.312271 76.372271) (width 0.3) (layer "B.Cu") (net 15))
 (segment (start 91.312271 76.372271) (end 91.04 76.372271) (width 0.3) (layer "B.Cu") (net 15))
 (segment (start 105.925 67.75) (end 103.125 70.55) (width 0.5) (layer "B.Cu") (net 15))
 (segment (start 91.296041 75.843959) (end 91.04 75.843959) (width 0.3) (layer "B.Cu") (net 15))
 (segment (start 91.25 75.797918) (end 91.296041 75.843959) (width 0.3) (layer "B.Cu") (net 15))
 (segment (start 86.155 95.02) (end 79.4 95.02) (width 0.5) (layer "B.Cu") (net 15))
 (segment (start 91.25 72.025) (end 91.25 75.797918) (width 0.5) (layer "B.Cu") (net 15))
 (segment (start 91.15 90.025) (end 86.155 95.02) (width 0.5) (layer "B.Cu") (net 15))
 (segment (start 92.725 70.55) (end 91.25 72.025) (width 0.5) (layer "B.Cu") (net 15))
 (segment (start 103.125 70.55) (end 92.725 70.55) (width 0.5) (layer "B.Cu") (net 15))
 (segment (start 91.15 76.534542) (end 91.15 90.025) (width 0.5) (layer "B.Cu") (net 15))
 (segment (start 82.7 66.615108) (end 87.265108 62.05) (width 0.3) (layer "F.Cu") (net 7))
 (segment (start 82.225 74.7) (end 82.7 74.225) (width 0.3) (layer "F.Cu") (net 7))
 (segment (start 87.265108 62.05) (end 93.275 62.05) (width 0.3) (layer "F.Cu") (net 7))
 (segment (start 79.4 74.7) (end 82.225 74.7) (width 0.3) (layer "F.Cu") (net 7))
 (segment (start 82.7 74.225) (end 82.7 66.615108) (width 0.3) (layer "F.Cu") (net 7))
 (via (at 93.275 62.05) (size 0.6) (drill 0.3) (layers "F.Cu" "B.Cu") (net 7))
 (segment (start 93.275 62.05) (end 93.275 55.555322) (width 0.3) (layer "B.Cu") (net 7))
 (segment (start 93.275 55.555322) (end 93.29 55.555322) (width 0.3) (layer "B.Cu") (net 7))
 (segment (start 81.75 69.9) (end 81.75 66.15) (width 0.3) (layer "F.Cu") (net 6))
 (segment (start 81.75 66.15) (end 86.825 61.075) (width 0.3) (layer "F.Cu") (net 6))
 (segment (start 79.49 72.16) (end 81.75 69.9) (width 0.3) (layer "F.Cu") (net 6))
 (segment (start 79.4 72.16) (end 79.49 72.16) (width 0.3) (layer "F.Cu") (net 6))
 (via (at 86.825 61.075) (size 0.6) (drill 0.3) (layers "F.Cu" "B.Cu") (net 6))
 (segment (start 90.75 59.85) (end 90.75 55.325) (width 0.3) (layer "B.Cu") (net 6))
 (segment (start 87 60.9) (end 89.7 60.9) (width 0.3) (layer "B.Cu") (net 6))
 (segment (start 89.7 60.9) (end 90.75 59.85) (width 0.3) (layer "B.Cu") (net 6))
 (segment (start 86.825 61.075) (end 87 60.9) (width 0.3) (layer "B.Cu") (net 6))
 (segment (start 64.7 98.522) (end 63.053 96.875) (width 0.3) (layer "F.Cu") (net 31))
 (segment (start 64.7 102.875) (end 64.7 98.522) (width 0.3) (layer "F.Cu") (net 31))
 (segment (start 61.2 102.875) (end 61.2 98.265) (width 0.3) (layer "F.Cu") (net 33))
 (segment (start 61.2 98.265) (end 59.81 96.875) (width 0.3) (layer "F.Cu") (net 33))
 (segment (start 71.7 102.875) (end 71.7 99.036) (width 0.3) (layer "F.Cu") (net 35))
 (segment (start 71.7 99.036) (end 69.539 96.875) (width 0.3) (layer "F.Cu") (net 35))
 (segment (start 68.2 102.875) (end 68.2 98.779) (width 0.3) (layer "F.Cu") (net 41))
 (segment (start 68.2 98.779) (end 66.296 96.875) (width 0.3) (layer "F.Cu") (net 41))
 (segment (start 65.075 67.775) (end 65.075 83.99) (width 0.3) (layer "F.Cu") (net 32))
 (segment (start 66.26 66.59) (end 65.075 67.775) (width 0.3) (layer "F.Cu") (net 32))
 (segment (start 69.27 66.59) (end 66.26 66.59) (width 0.3) (layer "F.Cu") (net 32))
 (segment (start 65.075 83.99) (end 59.81 89.255) (width 0.3) (layer "F.Cu") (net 32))
 (segment (start 67.445 69.13) (end 65.925 70.65) (width 0.3) (layer "F.Cu") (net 30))
 (segment (start 65.925 70.65) (end 65.925 86.383) (width 0.3) (layer "F.Cu") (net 30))
 (segment (start 65.925 86.383) (end 63.053 89.255) (width 0.3) (layer "F.Cu") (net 30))
 (segment (start 69.27 69.13) (end 67.445 69.13) (width 0.3) (layer "F.Cu") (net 30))
 (segment (start 66.825 72.9) (end 66.825 88.726) (width 0.3) (layer "F.Cu") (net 40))
 (segment (start 66.825 88.726) (end 66.296 89.255) (width 0.3) (layer "F.Cu") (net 40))
 (segment (start 68.055 71.67) (end 66.825 72.9) (width 0.3) (layer "F.Cu") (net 40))
 (segment (start 69.27 71.67) (end 68.055 71.67) (width 0.3) (layer "F.Cu") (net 40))
 (segment (start 67.619 87.335) (end 69.539 89.255) (width 0.3) (layer "F.Cu") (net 34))
 (segment (start 69.27 74.21) (end 67.619 75.861) (width 0.3) (layer "F.Cu") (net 34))
 (segment (start 67.619 75.861) (end 67.619 87.335) (width 0.3) (layer "F.Cu") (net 34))
 (segment (start 72.782 77.832) (end 71.7 76.75) (width 0.3) (layer "F.Cu") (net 38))
 (segment (start 72.782 89.255) (end 72.782 77.832) (width 0.3) (layer "F.Cu") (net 38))
 (segment (start 71.7 76.75) (end 69.27 76.75) (width 0.3) (layer "F.Cu") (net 38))
 (segment (start 70.91 79.29) (end 70.925 79.275) (width 0.3) (layer "F.Cu") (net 36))
 (segment (start 69.27 79.29) (end 70.91 79.29) (width 0.3) (layer "F.Cu") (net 36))
 (via (at 70.925 79.275) (size 0.6) (drill 0.3) (layers "F.Cu" "B.Cu") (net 36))
 (segment (start 70.925 79.275) (end 74.4 79.275) (width 0.3) (layer "B.Cu") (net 36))
 (segment (start 74.4 79.275) (end 75.975 80.85) (width 0.3) (layer "B.Cu") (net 36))
 (segment (start 75.975 88.921387) (end 76.025 88.921387) (width 0.3) (layer "B.Cu") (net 36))
 (segment (start 75.975 80.85) (end 75.975 88.921387) (width 0.3) (layer "B.Cu") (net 36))
 (segment (start 75.2 102.875) (end 75.2 99.293) (width 0.3) (layer "F.Cu") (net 39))
 (segment (start 75.2 99.293) (end 72.782 96.875) (width 0.3) (layer "F.Cu") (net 39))
 (segment (start 78.7 102.875) (end 78.7 99.55) (width 0.3) (layer "F.Cu") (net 37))
 (segment (start 78.7 99.55) (end 76.025 96.875) (width 0.3) (layer "F.Cu") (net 37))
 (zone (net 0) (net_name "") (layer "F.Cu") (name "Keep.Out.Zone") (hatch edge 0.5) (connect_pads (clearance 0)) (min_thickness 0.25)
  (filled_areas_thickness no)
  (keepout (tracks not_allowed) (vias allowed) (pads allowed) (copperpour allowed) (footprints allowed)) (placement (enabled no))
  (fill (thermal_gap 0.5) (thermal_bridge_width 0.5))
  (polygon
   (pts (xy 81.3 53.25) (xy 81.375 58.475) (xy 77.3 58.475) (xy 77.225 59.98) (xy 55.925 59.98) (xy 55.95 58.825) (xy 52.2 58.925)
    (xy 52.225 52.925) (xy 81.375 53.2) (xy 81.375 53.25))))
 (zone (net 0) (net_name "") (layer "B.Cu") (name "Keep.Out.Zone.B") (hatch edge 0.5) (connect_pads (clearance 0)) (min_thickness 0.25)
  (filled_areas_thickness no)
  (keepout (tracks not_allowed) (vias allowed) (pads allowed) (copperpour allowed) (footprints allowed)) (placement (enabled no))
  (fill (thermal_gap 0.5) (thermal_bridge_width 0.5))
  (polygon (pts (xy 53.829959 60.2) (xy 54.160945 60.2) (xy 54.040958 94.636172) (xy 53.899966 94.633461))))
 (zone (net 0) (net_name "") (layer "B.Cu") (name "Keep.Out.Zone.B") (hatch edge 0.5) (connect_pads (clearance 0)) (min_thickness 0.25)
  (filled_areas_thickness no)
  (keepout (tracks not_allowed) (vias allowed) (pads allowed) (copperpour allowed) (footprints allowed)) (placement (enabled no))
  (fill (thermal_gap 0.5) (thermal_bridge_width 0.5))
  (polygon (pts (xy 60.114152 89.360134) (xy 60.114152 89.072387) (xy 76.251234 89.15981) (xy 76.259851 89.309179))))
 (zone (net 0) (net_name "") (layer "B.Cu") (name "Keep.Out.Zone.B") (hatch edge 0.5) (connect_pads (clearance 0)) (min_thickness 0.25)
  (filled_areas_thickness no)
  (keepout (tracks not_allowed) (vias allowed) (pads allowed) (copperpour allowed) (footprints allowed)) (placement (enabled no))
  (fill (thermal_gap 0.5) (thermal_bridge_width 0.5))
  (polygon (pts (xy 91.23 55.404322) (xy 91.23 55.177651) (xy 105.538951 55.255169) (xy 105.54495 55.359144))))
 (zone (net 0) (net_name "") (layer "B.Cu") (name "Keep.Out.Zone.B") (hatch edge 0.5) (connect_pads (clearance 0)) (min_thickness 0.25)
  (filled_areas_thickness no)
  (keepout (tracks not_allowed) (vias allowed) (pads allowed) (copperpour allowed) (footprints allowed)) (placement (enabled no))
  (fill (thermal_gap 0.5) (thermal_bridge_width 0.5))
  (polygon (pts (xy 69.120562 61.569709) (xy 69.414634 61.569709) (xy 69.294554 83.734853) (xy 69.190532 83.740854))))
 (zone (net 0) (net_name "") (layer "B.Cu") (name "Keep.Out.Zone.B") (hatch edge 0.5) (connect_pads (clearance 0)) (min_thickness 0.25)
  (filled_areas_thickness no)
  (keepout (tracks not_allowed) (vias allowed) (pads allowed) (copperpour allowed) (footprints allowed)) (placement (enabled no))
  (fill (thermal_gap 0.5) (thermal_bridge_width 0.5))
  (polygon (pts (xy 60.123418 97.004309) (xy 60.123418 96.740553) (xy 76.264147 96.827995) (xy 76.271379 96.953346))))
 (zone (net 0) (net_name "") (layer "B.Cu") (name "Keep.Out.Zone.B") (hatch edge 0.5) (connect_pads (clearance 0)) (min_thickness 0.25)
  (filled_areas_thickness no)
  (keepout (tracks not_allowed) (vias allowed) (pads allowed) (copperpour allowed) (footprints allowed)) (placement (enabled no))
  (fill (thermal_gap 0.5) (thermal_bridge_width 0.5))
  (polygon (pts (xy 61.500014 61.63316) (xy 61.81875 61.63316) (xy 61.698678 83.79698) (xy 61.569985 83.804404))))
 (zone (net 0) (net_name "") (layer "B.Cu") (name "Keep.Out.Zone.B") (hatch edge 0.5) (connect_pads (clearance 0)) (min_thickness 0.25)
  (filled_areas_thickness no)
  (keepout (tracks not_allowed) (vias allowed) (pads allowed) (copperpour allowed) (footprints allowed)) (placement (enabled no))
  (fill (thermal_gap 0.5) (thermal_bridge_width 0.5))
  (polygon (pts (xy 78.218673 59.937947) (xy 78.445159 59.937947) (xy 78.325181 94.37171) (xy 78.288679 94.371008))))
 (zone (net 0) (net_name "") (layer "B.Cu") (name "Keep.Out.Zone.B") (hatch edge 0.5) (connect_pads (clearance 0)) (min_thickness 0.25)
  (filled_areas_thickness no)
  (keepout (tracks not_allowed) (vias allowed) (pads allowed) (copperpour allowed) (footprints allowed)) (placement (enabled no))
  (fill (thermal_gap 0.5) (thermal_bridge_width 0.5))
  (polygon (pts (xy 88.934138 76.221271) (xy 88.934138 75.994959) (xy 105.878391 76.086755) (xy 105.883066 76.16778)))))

